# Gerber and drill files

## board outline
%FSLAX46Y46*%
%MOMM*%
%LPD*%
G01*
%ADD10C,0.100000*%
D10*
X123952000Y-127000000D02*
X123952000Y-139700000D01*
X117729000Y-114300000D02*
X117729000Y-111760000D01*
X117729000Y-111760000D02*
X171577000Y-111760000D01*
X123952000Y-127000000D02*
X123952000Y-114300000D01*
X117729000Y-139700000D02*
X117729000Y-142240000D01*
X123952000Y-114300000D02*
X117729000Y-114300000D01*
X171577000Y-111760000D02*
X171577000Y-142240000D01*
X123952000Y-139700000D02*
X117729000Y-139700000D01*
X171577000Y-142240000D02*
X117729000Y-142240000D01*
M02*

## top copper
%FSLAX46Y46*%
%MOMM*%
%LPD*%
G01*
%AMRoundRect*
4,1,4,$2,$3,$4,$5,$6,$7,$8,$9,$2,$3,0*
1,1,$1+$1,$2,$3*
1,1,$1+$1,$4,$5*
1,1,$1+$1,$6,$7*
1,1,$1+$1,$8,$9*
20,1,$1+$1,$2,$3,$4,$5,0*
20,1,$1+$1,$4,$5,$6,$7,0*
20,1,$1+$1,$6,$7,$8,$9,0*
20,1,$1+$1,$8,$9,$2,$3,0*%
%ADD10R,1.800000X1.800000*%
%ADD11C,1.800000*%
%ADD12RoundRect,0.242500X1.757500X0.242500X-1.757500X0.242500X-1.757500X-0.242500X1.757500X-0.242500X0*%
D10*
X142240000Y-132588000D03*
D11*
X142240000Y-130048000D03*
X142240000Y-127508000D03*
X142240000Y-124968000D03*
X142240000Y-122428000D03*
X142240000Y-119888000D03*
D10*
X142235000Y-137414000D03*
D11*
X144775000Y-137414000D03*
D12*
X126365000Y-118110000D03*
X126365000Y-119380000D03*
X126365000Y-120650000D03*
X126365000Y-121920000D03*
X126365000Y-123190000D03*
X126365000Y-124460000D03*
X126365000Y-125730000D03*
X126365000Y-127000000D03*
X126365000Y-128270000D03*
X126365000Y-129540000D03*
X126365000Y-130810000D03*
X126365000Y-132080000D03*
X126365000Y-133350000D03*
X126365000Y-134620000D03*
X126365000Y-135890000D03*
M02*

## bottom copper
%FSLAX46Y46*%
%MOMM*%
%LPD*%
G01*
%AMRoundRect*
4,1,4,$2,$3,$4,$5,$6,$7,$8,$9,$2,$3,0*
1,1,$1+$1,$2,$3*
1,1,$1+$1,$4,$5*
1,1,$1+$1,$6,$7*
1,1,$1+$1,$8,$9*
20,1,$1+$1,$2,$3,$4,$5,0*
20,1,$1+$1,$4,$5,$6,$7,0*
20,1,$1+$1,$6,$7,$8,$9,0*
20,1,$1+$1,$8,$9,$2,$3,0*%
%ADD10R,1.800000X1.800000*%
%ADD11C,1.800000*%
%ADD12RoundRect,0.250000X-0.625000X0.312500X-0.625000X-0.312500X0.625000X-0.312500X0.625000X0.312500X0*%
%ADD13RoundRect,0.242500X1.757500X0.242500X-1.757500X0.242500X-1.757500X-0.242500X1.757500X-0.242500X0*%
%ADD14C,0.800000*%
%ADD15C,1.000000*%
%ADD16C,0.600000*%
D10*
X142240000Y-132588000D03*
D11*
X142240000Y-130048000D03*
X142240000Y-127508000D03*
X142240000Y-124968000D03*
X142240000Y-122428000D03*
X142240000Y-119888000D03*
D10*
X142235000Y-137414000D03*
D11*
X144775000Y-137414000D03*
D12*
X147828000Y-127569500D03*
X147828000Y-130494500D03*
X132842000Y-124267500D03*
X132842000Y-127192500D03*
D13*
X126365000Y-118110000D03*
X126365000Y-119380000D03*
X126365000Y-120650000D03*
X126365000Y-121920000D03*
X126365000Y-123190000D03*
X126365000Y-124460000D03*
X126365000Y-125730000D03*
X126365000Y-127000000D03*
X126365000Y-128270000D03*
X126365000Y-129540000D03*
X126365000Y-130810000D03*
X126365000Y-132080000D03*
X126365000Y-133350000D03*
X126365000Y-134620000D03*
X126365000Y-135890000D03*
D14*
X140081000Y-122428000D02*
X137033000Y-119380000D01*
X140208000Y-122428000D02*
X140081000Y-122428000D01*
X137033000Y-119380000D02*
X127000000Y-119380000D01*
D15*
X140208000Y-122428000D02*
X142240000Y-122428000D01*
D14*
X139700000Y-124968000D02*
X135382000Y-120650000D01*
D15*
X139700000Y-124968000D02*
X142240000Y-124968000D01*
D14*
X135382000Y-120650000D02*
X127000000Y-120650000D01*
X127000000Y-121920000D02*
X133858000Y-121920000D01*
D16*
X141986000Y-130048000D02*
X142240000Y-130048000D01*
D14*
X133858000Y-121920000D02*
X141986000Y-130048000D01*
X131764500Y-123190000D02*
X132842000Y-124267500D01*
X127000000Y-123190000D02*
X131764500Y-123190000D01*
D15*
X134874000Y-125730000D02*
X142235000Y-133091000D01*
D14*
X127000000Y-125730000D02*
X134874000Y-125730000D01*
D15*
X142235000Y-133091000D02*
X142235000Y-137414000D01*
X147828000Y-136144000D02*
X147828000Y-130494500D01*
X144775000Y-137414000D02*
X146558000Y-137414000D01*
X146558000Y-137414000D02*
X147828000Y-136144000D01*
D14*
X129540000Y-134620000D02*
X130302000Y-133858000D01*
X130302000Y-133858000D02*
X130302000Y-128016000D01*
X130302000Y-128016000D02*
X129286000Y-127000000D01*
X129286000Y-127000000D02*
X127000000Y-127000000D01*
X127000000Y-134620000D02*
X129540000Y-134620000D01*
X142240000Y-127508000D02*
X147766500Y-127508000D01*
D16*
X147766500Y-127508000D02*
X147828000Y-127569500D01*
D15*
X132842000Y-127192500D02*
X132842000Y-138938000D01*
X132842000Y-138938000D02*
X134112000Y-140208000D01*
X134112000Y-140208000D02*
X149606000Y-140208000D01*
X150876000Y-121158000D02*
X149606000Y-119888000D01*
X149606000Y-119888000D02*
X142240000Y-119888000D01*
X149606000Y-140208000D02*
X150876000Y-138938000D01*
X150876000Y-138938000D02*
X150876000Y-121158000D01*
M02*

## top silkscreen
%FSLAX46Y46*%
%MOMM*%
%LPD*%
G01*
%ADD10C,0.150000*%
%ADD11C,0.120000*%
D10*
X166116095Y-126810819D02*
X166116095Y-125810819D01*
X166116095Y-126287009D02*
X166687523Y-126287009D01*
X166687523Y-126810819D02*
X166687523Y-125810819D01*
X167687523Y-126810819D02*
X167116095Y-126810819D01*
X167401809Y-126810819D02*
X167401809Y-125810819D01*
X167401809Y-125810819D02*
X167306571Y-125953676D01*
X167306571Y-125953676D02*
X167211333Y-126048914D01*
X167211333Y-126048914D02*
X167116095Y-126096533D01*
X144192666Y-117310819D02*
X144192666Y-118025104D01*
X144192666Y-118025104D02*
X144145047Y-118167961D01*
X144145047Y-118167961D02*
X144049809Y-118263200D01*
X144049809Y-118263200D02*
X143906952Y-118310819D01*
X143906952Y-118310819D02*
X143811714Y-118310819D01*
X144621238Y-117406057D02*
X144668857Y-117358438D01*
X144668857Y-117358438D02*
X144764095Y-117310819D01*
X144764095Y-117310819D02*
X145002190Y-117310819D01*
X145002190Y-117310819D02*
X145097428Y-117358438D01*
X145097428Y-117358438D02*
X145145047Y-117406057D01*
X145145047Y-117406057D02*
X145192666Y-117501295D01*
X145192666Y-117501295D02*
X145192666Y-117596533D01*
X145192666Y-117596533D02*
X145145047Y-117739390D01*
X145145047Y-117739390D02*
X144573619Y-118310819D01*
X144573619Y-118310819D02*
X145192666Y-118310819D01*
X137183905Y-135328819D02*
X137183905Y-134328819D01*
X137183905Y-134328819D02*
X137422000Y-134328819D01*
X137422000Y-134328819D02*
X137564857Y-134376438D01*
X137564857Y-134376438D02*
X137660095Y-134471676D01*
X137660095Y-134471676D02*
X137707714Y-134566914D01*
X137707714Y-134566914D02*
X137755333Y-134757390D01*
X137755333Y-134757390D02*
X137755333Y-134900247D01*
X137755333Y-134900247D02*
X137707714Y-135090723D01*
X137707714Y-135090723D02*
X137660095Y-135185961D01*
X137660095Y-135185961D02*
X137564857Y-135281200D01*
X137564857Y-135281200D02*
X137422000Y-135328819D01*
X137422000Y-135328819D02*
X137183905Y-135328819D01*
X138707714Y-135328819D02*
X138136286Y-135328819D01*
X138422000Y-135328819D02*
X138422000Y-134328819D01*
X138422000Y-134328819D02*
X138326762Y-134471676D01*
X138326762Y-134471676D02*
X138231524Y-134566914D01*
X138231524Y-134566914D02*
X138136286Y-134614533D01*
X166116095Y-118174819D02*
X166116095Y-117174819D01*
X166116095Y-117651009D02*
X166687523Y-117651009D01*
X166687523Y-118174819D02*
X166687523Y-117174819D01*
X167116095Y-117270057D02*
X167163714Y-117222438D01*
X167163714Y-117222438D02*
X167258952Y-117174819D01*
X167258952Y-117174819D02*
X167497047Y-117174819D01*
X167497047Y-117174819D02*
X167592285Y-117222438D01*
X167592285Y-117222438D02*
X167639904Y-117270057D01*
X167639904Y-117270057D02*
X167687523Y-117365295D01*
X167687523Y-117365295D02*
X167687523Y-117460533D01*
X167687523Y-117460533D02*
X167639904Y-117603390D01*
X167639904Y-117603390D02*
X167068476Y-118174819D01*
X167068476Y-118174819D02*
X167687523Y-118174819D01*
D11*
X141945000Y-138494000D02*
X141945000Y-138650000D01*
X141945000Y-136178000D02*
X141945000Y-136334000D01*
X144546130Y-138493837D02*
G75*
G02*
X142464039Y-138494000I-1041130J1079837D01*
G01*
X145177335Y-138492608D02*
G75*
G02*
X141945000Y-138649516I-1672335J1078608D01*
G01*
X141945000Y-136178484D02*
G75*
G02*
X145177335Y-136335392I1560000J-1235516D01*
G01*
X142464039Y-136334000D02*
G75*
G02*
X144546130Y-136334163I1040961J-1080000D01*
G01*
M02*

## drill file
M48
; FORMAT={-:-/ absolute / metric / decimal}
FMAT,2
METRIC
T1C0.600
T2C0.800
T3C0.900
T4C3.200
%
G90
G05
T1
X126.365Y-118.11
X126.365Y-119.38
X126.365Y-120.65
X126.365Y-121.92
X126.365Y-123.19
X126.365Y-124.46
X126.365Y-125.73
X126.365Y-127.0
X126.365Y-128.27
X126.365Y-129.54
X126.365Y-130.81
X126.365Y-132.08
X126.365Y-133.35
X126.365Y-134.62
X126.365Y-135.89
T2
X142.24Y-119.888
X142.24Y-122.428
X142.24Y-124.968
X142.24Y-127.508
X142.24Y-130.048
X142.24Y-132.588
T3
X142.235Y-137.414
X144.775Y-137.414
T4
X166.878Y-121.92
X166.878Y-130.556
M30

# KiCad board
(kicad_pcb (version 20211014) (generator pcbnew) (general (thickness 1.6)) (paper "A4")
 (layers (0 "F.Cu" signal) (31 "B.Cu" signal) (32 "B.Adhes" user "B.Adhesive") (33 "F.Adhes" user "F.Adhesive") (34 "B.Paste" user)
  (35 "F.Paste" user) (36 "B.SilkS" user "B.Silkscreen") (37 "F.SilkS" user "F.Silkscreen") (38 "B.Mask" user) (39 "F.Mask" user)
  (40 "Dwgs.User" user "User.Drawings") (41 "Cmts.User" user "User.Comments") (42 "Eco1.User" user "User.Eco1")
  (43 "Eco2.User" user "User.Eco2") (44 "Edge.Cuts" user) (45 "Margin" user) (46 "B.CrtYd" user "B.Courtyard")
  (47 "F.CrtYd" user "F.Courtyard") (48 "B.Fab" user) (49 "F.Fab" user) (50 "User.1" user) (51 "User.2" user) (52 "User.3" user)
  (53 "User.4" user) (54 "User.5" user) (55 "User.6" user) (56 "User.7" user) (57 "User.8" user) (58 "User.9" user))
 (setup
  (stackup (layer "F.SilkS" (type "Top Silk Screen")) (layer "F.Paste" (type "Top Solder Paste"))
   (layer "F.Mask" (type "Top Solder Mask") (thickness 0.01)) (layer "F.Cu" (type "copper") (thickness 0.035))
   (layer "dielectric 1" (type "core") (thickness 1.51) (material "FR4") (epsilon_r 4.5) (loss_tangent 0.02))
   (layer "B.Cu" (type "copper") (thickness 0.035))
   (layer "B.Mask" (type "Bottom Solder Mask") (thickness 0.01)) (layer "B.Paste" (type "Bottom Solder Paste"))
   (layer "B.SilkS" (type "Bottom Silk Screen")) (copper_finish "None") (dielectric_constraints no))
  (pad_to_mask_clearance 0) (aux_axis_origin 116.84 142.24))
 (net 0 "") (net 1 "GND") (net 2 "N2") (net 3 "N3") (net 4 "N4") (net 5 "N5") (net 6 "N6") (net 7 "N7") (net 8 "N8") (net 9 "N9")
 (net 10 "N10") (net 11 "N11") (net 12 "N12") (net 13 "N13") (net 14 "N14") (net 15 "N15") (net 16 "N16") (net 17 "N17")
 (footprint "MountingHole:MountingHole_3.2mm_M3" (layer "F.Cu") (at 166.878 130.556)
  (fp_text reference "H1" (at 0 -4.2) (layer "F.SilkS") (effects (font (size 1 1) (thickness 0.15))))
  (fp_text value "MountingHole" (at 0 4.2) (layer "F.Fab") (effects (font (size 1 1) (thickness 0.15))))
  (pad "" np_thru_hole circle locked (at 0 0) (size 3.2 3.2) (drill 3.2) (layers *.Cu *.Mask)))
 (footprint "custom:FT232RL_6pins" (layer "F.Cu") (at 142.24 132.588 180)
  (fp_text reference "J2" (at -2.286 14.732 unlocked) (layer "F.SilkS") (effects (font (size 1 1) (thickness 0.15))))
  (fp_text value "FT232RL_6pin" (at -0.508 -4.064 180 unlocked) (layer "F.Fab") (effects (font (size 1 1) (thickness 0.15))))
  (pad "1" thru_hole rect (at 0 0 180) (size 1.8 1.8) (drill 0.8) (layers *.Cu *.Mask) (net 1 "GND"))
  (pad "2" thru_hole circle (at 0 2.54 180) (size 1.8 1.8) (drill 0.8) (layers *.Cu *.Mask) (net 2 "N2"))
  (pad "3" thru_hole circle (at 0 5.08 180) (size 1.8 1.8) (drill 0.8) (layers *.Cu *.Mask) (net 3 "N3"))
  (pad "4" thru_hole circle (at 0 7.62 180) (size 1.8 1.8) (drill 0.8) (layers *.Cu *.Mask) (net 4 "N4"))
  (pad "5" thru_hole circle (at 0 10.16 180) (size 1.8 1.8) (drill 0.8) (layers *.Cu *.Mask) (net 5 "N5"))
  (pad "6" thru_hole circle (at 0 12.7 180) (size 1.8 1.8) (drill 0.8) (layers *.Cu *.Mask) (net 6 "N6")))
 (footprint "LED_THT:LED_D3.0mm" (layer "F.Cu") (at 142.235 137.414)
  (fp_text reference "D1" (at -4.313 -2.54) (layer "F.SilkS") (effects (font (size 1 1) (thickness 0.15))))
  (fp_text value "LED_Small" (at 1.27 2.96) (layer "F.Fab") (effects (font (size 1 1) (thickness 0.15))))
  (fp_line (start -0.29 1.08) (end -0.29 1.236) (layer "F.SilkS") (width 0.12))
  (fp_line (start -0.29 -1.236) (end -0.29 -1.08) (layer "F.SilkS") (width 0.12))
  (fp_arc (start 2.31113 1.079837) (mid 1.270117 1.5) (end 0.229039 1.08) (layer "F.SilkS") (width 0.12))
  (fp_arc (start 2.942335 1.078608) (mid 1.366487 1.987659) (end -0.29 1.235516) (layer "F.SilkS") (width 0.12))
  (fp_arc (start -0.29 -1.235516) (mid 1.366487 -1.987659) (end 2.942335 -1.078608) (layer "F.SilkS") (width 0.12))
  (fp_arc (start 0.229039 -1.08) (mid 1.270117 -1.5) (end 2.31113 -1.079837) (layer "F.SilkS") (width 0.12))
  (pad "1" thru_hole rect locked (at 0 0) (size 1.8 1.8) (drill 0.9) (layers *.Cu *.Mask) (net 1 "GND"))
  (pad "2" thru_hole circle locked (at 2.54 0) (size 1.8 1.8) (drill 0.9) (layers *.Cu *.Mask) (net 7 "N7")))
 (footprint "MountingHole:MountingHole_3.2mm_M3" (layer "F.Cu") (at 166.878 121.92)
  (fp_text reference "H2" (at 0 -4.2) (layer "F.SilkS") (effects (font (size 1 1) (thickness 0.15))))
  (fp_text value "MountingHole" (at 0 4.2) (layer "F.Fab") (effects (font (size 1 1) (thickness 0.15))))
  (pad "" np_thru_hole circle locked (at 0 0) (size 3.2 3.2) (drill 3.2) (layers *.Cu *.Mask)))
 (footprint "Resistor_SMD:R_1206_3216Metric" (layer "B.Cu") (at 147.828 129.032 -90)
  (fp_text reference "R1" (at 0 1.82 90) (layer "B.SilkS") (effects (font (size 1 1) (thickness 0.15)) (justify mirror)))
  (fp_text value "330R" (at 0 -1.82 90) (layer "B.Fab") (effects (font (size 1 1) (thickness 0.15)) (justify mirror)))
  (pad "1" smd roundrect locked (at -1.4625 0 270) (size 1.125 1.75) (layers "B.Cu" "B.Paste" "B.Mask") (roundrect_rratio 0.222222)
   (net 3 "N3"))
  (pad "2" smd roundrect locked (at 1.4625 0 270) (size 1.125 1.75) (layers "B.Cu" "B.Paste" "B.Mask") (roundrect_rratio 0.222222)
   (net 7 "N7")))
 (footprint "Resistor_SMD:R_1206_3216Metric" (layer "B.Cu") (at 132.842 125.73 -90)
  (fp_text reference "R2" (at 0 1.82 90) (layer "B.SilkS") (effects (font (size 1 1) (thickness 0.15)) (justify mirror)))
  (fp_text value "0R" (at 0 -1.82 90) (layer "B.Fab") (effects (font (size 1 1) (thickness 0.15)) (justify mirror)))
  (pad "1" smd roundrect locked (at -1.4625 0 270) (size 1.125 1.75) (layers "B.Cu" "B.Paste" "B.Mask") (roundrect_rratio 0.222222)
   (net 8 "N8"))
  (pad "2" smd roundrect locked (at 1.4625 0 270) (size 1.125 1.75) (layers "B.Cu" "B.Paste" "B.Mask") (roundrect_rratio 0.222222)
   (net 6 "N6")))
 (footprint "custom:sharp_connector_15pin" (layer "B.Cu") (at 126.365 127 180)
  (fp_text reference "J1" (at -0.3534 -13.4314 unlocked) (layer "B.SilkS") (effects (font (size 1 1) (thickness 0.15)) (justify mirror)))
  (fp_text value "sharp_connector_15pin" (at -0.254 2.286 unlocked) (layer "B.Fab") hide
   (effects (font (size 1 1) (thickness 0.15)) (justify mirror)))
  (pad "1" thru_hole roundrect (at 0 8.89 180) (size 4 0.97) (drill 0.6) (layers *.Cu *.Mask) (roundrect_rratio 0.25) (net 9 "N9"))
  (pad "2" thru_hole roundrect (at 0 7.62 180) (size 4 0.97) (drill 0.6) (layers *.Cu *.Mask) (roundrect_rratio 0.25) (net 5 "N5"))
  (pad "3" thru_hole roundrect (at 0 6.35 180) (size 4 0.97) (drill 0.6) (layers *.Cu *.Mask) (roundrect_rratio 0.25) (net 4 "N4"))
  (pad "4" thru_hole roundrect (at 0 5.08 180) (size 4 0.97) (drill 0.6) (layers *.Cu *.Mask) (roundrect_rratio 0.25) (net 2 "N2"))
  (pad "5" thru_hole roundrect (at 0 3.81 180) (size 4 0.97) (drill 0.6) (layers *.Cu *.Mask) (roundrect_rratio 0.25) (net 8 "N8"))
  (pad "6" thru_hole roundrect (at 0 2.54 180) (size 4 0.97) (drill 0.6) (layers *.Cu *.Mask) (roundrect_rratio 0.25) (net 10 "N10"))
  (pad "7" thru_hole roundrect (at 0 1.27 180) (size 4 0.97) (drill 0.6) (layers *.Cu *.Mask) (roundrect_rratio 0.25) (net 1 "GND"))
  (pad "8" thru_hole roundrect (at 0 0 180) (size 4 0.97) (drill 0.6) (layers *.Cu *.Mask) (roundrect_rratio 0.25) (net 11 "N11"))
  (pad "9" thru_hole roundrect (at 0 -1.27 180) (size 4 0.97) (drill 0.6) (layers *.Cu *.Mask) (roundrect_rratio 0.25) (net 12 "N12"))
  (pad "10" thru_hole roundrect (at 0 -2.54 180) (size 4 0.97) (drill 0.6) (layers *.Cu *.Mask) (roundrect_rratio 0.25) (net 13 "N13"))
  (pad "11" thru_hole roundrect (at 0 -3.81 180) (size 4 0.97) (drill 0.6) (layers *.Cu *.Mask) (roundrect_rratio 0.25) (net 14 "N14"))
  (pad "12" thru_hole roundrect (at 0 -5.08 180) (size 4 0.97) (drill 0.6) (layers *.Cu *.Mask) (roundrect_rratio 0.25) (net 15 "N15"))
  (pad "13" thru_hole roundrect (at 0 -6.35 180) (size 4 0.97) (drill 0.6) (layers *.Cu *.Mask) (roundrect_rratio 0.25) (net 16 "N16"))
  (pad "14" thru_hole roundrect (at 0 -7.62 180) (size 4 0.97) (drill 0.6) (layers *.Cu *.Mask) (roundrect_rratio 0.25) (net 11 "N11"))
  (pad "15" thru_hole roundrect (at 0 -8.89 180) (size 4 0.97) (drill 0.6) (layers *.Cu *.Mask) (roundrect_rratio 0.25) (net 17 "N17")))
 (gr_line (start 123.952 127) (end 123.952 139.7) (layer "Edge.Cuts") (width 0.1))
 (gr_line (start 117.729 114.3) (end 117.729 111.76) (layer "Edge.Cuts") (width 0.1))
 (gr_line (start 117.729 111.76) (end 171.577 111.76) (layer "Edge.Cuts") (width 0.1))
 (gr_line (start 123.952 127) (end 123.952 114.3) (layer "Edge.Cuts") (width 0.1))
 (gr_line (start 117.729 139.7) (end 117.729 142.24) (layer "Edge.Cuts") (width 0.1))
 (gr_line (start 123.952 114.3) (end 117.729 114.3) (layer "Edge.Cuts") (width 0.1))
 (gr_line (start 171.577 111.76) (end 171.577 142.24) (layer "Edge.Cuts") (width 0.1))
 (gr_line (start 123.952 139.7) (end 117.729 139.7) (layer "Edge.Cuts") (width 0.1))
 (gr_line (start 171.577 142.24) (end 117.729 142.24) (layer "Edge.Cuts") (width 0.1))
 (segment (start 140.081 122.428) (end 137.033 119.38) (width 0.8) (layer "B.Cu") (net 5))
 (segment (start 140.208 122.428) (end 140.081 122.428) (width 0.8) (layer "B.Cu") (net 5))
 (segment (start 137.033 119.38) (end 127 119.38) (width 0.8) (layer "B.Cu") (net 5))
 (segment (start 140.208 122.428) (end 142.24 122.428) (width 1) (layer "B.Cu") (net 5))
 (segment (start 139.7 124.968) (end 135.382 120.65) (width 0.8) (layer "B.Cu") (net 4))
 (segment (start 139.7 124.968) (end 142.24 124.968) (width 1) (layer "B.Cu") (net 4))
 (segment (start 135.382 120.65) (end 127 120.65) (width 0.8) (layer "B.Cu") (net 4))
 (segment (start 127 121.92) (end 133.858 121.92) (width 0.8) (layer "B.Cu") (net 2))
 (segment (start 141.986 130.048) (end 142.24 130.048) (width 0.6) (layer "B.Cu") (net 2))
 (segment (start 133.858 121.92) (end 141.986 130.048) (width 0.8) (layer "B.Cu") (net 2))
 (segment (start 131.7645 123.19) (end 132.842 124.2675) (width 0.8) (layer "B.Cu") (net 8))
 (segment (start 127 123.19) (end 131.7645 123.19) (width 0.8) (layer "B.Cu") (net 8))
 (segment (start 134.874 125.73) (end 142.235 133.091) (width 1) (layer "B.Cu") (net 1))
 (segment (start 127 125.73) (end 134.874 125.73) (width 0.8) (layer "B.Cu") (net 1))
 (segment (start 142.235 133.091) (end 142.235 137.414) (width 1) (layer "B.Cu") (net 1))
 (segment (start 147.828 136.144) (end 147.828 130.4945) (width 1) (layer "B.Cu") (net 7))
 (segment (start 144.775 137.414) (end 146.558 137.414) (width 1) (layer "B.Cu") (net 7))
 (segment (start 146.558 137.414) (end 147.828 136.144) (width 1) (layer "B.Cu") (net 7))
 (segment (start 129.54 134.62) (end 130.302 133.858) (width 0.8) (layer "B.Cu") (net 11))
 (segment (start 130.302 133.858) (end 130.302 128.016) (width 0.8) (layer "B.Cu") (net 11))
 (segment (start 130.302 128.016) (end 129.286 127) (width 0.8) (layer "B.Cu") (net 11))
 (segment (start 129.286 127) (end 127 127) (width 0.8) (layer "B.Cu") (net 11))
 (segment (start 127 134.62) (end 129.54 134.62) (width 0.8) (layer "B.Cu") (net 11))
 (segment (start 142.24 127.508) (end 147.7665 127.508) (width 0.8) (layer "B.Cu") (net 3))
 (segment (start 147.7665 127.508) (end 147.828 127.5695) (width 0.6) (layer "B.Cu") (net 3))
 (segment (start 132.842 127.1925) (end 132.842 138.938) (width 1) (layer "B.Cu") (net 6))
 (segment (start 132.842 138.938) (end 134.112 140.208) (width 1) (layer "B.Cu") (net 6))
 (segment (start 134.112 140.208) (end 149.606 140.208) (width 1) (layer "B.Cu") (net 6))
 (segment (start 150.876 121.158) (end 149.606 119.888) (width 1) (layer "B.Cu") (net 6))
 (segment (start 149.606 119.888) (end 142.24 119.888) (width 1) (layer "B.Cu") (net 6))
 (segment (start 149.606 140.208) (end 150.876 138.938) (width 1) (layer "B.Cu") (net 6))
 (segment (start 150.876 138.938) (end 150.876 121.158) (width 1) (layer "B.Cu") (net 6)))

